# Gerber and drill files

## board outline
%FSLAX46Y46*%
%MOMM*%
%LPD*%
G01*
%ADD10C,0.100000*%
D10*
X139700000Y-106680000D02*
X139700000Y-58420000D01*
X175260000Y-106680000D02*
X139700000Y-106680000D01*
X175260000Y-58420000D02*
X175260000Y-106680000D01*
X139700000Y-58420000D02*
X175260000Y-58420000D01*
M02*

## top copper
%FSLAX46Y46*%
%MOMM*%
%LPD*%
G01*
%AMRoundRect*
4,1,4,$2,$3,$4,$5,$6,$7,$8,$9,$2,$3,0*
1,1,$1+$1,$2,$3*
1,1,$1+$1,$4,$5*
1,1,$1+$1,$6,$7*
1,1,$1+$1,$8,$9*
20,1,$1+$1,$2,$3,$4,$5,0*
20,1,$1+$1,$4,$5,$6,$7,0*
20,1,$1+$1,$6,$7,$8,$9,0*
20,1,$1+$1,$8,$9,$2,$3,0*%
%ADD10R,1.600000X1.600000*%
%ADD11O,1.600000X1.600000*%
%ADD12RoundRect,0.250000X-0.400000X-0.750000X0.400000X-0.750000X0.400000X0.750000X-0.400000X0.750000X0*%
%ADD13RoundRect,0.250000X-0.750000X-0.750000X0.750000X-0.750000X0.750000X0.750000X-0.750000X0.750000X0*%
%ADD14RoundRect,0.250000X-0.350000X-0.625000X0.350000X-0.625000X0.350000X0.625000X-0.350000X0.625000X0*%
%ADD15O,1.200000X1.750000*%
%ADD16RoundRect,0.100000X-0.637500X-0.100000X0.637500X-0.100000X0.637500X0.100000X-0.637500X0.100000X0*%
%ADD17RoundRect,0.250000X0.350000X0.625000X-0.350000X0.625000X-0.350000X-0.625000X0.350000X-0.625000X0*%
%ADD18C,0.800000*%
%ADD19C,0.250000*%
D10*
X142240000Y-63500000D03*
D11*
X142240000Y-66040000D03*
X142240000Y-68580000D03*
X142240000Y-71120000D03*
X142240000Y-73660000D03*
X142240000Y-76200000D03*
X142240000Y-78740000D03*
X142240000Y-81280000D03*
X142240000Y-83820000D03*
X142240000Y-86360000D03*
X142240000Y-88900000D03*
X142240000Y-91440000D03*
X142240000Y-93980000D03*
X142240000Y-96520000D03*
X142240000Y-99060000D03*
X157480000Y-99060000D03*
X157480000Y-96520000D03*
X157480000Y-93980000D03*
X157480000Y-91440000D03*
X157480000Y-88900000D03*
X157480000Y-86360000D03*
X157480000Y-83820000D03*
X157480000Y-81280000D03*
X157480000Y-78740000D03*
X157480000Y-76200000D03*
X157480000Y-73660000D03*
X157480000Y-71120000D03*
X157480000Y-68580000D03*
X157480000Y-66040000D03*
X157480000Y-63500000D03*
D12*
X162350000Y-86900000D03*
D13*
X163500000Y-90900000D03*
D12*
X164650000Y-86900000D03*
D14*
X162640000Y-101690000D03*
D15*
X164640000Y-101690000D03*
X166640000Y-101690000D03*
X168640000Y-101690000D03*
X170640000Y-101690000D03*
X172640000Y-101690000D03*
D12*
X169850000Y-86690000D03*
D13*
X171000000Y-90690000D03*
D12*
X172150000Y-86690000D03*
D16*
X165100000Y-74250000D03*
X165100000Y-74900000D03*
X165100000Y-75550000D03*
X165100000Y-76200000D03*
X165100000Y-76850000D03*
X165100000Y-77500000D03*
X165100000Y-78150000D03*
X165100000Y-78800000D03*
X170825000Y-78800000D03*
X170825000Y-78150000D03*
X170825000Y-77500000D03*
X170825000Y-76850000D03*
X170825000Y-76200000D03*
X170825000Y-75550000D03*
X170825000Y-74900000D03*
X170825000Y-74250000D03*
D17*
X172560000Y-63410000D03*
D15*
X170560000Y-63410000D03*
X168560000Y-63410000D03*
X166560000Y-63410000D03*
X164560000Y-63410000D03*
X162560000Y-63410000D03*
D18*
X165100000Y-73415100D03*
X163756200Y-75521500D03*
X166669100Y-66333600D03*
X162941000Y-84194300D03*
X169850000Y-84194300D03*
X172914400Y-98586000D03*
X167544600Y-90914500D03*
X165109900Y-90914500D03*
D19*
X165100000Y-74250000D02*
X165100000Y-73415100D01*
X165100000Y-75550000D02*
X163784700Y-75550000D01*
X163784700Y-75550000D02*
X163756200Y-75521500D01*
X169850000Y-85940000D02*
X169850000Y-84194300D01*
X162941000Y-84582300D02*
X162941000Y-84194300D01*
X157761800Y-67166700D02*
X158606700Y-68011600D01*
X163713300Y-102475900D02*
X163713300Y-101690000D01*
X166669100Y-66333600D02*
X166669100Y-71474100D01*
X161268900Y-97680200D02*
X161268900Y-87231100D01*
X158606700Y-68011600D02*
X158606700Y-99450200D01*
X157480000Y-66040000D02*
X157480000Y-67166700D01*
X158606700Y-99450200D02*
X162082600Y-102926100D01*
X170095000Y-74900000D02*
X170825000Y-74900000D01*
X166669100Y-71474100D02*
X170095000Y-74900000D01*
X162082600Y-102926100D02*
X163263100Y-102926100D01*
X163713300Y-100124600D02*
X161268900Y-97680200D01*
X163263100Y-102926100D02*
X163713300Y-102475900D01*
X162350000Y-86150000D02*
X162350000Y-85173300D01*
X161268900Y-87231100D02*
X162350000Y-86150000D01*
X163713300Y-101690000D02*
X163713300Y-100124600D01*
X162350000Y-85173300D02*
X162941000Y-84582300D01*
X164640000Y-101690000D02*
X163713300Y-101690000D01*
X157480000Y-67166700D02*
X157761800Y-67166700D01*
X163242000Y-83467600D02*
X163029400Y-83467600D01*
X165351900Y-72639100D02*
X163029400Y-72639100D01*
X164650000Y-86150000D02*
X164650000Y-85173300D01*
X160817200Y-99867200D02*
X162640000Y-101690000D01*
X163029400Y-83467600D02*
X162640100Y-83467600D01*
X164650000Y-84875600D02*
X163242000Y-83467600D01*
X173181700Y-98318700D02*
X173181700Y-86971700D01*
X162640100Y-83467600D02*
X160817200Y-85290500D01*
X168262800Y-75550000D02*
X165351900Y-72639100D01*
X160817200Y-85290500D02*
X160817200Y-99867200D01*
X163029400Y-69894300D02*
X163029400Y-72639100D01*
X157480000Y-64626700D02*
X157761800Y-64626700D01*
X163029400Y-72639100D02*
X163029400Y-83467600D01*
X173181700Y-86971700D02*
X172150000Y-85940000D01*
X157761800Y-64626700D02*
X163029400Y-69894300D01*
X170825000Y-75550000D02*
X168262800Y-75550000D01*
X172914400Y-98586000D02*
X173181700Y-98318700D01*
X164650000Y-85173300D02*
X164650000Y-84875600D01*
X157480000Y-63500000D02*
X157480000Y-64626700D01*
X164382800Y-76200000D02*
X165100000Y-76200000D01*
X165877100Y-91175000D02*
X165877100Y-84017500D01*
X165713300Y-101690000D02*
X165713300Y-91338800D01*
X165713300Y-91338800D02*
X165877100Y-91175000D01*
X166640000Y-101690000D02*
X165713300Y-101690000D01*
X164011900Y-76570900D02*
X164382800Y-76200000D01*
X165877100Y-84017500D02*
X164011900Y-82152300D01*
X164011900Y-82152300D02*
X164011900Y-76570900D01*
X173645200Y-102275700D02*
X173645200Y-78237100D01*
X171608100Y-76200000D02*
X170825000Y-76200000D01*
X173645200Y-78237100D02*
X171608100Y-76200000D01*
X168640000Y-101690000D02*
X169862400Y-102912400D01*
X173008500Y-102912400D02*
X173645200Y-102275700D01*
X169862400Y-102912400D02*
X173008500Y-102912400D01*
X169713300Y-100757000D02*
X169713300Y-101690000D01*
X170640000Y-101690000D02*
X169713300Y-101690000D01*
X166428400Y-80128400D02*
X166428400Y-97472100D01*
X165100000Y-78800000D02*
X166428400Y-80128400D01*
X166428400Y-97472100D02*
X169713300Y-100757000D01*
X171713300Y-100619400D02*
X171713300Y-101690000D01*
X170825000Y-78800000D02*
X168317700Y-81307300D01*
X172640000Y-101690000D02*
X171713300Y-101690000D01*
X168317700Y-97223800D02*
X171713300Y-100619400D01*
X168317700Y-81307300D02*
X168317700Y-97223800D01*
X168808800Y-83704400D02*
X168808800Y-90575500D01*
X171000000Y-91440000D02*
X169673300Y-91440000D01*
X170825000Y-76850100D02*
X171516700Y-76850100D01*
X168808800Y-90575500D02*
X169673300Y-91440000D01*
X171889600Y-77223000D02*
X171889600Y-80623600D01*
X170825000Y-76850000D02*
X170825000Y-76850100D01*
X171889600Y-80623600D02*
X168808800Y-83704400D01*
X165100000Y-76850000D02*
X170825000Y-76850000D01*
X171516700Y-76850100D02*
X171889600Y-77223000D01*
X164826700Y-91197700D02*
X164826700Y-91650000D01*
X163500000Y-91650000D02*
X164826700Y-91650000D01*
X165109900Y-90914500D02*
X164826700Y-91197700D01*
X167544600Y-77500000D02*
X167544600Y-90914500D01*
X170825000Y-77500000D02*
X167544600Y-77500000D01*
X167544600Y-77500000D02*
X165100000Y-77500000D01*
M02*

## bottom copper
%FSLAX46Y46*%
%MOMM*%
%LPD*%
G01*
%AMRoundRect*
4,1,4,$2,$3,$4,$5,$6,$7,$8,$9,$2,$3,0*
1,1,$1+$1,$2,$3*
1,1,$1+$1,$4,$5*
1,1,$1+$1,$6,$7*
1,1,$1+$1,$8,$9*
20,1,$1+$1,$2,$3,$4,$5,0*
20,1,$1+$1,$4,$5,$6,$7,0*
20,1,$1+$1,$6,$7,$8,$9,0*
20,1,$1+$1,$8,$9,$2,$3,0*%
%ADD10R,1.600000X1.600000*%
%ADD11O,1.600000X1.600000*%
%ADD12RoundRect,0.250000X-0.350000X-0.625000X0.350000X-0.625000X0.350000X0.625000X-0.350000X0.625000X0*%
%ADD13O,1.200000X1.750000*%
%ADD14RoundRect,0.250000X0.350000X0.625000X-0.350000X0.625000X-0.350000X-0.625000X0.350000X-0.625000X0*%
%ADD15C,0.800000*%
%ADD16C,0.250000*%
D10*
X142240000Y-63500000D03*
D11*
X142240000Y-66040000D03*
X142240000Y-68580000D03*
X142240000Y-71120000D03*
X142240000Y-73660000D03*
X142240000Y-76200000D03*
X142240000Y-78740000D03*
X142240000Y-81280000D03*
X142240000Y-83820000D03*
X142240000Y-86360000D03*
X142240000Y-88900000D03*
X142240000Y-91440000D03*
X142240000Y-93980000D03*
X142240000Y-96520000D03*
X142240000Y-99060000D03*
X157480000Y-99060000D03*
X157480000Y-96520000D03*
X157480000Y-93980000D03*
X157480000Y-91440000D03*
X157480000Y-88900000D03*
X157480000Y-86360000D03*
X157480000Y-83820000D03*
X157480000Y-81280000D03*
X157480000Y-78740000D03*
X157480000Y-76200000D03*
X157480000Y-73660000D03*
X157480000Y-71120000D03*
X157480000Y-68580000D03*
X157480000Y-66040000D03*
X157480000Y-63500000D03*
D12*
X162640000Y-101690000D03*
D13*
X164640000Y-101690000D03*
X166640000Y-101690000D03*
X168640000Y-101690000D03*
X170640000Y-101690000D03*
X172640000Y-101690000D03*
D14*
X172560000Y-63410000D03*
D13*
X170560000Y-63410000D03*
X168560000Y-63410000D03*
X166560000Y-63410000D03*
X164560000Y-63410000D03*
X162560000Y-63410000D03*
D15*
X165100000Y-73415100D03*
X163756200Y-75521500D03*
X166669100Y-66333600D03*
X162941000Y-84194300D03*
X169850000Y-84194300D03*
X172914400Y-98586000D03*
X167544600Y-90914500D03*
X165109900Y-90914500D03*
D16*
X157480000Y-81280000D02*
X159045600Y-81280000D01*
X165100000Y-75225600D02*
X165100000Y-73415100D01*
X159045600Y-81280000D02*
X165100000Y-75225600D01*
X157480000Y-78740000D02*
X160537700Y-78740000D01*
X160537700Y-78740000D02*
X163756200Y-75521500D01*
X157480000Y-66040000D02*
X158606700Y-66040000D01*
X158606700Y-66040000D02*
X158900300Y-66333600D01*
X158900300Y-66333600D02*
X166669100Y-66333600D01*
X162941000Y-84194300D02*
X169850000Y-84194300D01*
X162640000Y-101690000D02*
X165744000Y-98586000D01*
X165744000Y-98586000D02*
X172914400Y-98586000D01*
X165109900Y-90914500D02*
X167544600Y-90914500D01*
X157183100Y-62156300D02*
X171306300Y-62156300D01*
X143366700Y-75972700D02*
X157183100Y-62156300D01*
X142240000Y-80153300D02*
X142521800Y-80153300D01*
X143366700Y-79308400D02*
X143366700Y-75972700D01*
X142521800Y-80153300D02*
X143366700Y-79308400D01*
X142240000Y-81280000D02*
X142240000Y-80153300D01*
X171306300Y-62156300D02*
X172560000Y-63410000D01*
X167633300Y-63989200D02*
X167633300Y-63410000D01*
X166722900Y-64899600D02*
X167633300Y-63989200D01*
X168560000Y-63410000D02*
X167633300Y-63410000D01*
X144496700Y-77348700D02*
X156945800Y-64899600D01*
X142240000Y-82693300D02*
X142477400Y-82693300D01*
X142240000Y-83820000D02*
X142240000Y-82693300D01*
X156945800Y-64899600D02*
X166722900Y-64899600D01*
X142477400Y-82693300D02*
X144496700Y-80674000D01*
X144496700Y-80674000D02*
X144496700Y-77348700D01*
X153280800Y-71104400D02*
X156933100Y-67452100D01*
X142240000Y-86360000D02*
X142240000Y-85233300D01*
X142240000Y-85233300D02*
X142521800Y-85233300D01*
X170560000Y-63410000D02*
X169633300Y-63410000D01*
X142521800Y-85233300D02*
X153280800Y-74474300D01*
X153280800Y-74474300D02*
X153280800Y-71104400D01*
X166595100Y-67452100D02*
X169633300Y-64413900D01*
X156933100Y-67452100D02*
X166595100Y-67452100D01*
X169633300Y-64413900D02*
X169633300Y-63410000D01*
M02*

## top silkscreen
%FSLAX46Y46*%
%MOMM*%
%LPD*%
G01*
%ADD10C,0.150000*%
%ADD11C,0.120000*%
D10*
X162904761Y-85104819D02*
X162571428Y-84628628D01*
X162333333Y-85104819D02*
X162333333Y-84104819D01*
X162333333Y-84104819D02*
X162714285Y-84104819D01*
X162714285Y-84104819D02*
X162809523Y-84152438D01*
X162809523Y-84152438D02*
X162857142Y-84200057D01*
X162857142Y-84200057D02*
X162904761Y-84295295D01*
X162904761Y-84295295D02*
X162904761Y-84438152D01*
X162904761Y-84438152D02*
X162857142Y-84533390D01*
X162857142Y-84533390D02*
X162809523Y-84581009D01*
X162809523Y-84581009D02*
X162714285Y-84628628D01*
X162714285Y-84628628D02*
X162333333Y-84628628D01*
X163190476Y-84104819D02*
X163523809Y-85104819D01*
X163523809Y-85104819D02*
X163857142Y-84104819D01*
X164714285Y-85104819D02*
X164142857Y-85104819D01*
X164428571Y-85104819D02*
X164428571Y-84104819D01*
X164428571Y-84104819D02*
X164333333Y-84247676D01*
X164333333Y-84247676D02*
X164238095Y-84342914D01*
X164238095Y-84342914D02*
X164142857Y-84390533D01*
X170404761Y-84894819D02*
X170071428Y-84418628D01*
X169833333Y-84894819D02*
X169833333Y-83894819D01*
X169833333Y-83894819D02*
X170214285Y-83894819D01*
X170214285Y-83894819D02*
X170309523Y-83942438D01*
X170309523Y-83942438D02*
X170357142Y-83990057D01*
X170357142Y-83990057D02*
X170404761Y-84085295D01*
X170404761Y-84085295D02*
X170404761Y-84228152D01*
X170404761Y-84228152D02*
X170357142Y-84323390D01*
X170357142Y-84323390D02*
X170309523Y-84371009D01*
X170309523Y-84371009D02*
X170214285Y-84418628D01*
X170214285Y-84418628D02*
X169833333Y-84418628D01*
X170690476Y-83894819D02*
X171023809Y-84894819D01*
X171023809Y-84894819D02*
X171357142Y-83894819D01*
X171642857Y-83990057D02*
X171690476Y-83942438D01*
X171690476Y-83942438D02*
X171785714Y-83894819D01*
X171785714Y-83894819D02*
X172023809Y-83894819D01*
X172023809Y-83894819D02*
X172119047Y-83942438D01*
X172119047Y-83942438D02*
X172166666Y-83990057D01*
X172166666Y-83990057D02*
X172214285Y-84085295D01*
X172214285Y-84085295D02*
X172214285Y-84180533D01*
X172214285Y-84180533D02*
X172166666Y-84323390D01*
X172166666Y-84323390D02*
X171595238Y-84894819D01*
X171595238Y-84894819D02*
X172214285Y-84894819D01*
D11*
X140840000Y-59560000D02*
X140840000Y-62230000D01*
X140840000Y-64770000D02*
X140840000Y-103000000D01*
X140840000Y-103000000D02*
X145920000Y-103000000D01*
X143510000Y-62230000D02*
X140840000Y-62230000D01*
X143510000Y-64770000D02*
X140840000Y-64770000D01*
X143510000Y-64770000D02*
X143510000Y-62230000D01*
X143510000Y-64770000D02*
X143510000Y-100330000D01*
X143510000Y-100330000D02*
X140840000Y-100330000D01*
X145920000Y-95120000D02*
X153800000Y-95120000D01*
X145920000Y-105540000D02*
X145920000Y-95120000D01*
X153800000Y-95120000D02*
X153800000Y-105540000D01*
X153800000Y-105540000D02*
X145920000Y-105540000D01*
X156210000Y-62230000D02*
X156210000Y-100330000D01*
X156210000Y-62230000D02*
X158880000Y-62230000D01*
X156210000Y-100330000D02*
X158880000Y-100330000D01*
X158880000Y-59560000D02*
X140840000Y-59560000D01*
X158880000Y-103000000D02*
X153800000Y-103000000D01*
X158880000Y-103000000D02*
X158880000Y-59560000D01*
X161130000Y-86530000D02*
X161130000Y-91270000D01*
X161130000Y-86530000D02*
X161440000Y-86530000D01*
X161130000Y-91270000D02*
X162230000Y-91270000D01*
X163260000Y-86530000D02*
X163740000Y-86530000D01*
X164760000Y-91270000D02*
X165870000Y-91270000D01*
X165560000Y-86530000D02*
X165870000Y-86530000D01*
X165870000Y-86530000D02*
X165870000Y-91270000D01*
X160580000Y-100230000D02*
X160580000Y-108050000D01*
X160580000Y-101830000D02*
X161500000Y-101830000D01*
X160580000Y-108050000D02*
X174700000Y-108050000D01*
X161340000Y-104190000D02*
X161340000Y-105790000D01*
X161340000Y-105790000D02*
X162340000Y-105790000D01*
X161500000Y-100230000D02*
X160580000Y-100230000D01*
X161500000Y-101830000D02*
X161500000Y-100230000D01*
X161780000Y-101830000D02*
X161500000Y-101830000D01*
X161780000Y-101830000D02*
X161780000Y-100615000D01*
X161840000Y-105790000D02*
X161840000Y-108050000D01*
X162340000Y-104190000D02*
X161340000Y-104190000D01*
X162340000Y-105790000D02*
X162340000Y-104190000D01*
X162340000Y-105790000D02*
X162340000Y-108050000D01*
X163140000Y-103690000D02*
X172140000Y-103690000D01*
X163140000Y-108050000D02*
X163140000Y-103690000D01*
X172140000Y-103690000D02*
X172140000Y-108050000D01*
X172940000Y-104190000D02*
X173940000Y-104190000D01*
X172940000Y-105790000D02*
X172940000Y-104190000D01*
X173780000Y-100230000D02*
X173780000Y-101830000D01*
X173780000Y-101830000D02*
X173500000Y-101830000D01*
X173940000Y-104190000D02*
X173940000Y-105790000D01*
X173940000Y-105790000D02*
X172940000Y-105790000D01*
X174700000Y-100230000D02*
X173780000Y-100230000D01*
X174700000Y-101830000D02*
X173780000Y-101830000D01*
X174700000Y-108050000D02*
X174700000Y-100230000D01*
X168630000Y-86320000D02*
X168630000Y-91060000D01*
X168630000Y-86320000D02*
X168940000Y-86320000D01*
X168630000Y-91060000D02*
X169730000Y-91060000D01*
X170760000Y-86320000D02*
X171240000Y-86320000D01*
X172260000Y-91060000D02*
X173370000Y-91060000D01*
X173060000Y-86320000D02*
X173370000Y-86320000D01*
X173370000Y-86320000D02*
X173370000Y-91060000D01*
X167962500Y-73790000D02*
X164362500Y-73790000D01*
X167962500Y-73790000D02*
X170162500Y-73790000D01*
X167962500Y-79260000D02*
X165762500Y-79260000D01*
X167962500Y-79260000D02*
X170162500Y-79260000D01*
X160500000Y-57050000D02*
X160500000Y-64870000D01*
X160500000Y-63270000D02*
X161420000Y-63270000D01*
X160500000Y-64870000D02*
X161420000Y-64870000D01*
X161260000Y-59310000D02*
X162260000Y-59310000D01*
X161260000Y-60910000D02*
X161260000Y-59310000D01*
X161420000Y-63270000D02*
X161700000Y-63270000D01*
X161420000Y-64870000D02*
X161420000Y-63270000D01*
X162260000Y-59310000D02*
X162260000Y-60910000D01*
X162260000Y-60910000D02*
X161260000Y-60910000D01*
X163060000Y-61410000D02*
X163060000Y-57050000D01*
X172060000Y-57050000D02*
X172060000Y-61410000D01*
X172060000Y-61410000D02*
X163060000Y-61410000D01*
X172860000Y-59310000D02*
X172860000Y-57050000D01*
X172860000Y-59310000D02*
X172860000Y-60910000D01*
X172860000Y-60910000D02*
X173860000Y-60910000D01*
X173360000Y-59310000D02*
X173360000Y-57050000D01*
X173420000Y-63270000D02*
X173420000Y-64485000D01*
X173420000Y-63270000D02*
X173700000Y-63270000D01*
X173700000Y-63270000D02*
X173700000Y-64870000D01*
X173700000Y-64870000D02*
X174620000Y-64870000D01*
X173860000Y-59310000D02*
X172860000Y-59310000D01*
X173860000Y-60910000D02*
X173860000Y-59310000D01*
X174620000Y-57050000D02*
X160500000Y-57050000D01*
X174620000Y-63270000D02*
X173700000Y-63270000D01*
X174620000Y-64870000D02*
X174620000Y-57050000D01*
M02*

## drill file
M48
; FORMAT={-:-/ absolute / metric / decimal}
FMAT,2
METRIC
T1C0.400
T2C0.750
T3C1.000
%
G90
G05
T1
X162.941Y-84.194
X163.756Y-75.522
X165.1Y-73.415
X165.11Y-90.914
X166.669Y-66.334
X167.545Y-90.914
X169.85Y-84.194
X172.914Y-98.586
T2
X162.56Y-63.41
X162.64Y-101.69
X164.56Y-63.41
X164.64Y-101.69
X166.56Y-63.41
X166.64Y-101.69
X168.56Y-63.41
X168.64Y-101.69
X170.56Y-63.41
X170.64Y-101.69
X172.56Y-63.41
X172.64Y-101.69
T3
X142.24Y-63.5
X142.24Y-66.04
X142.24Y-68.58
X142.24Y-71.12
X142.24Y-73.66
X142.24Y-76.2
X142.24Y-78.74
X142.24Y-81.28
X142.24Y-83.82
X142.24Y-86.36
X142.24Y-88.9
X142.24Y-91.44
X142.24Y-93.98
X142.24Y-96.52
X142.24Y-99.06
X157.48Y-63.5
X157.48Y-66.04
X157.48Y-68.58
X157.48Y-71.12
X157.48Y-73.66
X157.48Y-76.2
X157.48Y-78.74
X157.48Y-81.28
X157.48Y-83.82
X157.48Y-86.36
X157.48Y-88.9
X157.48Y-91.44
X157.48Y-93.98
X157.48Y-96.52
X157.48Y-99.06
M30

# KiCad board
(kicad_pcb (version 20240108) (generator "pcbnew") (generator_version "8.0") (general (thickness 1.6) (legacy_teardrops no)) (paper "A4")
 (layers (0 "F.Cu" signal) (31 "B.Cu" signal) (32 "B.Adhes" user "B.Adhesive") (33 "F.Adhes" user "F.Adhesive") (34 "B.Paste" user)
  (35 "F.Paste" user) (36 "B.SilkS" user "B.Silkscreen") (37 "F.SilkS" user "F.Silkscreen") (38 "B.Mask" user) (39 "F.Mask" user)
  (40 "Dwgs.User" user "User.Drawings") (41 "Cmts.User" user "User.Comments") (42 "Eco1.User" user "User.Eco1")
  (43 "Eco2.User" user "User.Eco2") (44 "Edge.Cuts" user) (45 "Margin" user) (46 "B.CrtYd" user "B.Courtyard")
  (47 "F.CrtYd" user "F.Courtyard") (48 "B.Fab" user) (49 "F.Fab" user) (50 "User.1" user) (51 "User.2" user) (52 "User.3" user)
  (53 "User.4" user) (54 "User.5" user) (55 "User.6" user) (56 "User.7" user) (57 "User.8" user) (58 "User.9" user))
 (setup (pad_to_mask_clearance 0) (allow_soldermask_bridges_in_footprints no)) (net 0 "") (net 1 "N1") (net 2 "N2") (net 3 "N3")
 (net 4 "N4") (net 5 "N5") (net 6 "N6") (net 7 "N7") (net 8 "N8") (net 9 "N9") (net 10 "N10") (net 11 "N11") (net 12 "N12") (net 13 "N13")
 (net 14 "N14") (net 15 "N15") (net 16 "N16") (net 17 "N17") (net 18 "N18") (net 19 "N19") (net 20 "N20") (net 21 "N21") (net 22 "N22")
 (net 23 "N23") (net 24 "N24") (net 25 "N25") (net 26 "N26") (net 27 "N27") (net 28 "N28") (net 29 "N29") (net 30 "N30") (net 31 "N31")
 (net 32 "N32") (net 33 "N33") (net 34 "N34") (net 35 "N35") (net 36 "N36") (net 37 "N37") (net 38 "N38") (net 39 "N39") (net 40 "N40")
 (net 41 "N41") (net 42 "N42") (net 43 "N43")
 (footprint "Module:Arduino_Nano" (layer "F.Cu") (at 142.24 63.5)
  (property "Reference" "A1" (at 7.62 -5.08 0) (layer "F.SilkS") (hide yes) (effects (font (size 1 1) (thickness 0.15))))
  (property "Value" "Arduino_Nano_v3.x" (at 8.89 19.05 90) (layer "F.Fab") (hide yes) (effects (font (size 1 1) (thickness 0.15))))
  (fp_line (start -1.4 -3.94) (end -1.4 -1.27) (stroke (width 0.12) (type solid)) (layer "F.SilkS"))
  (fp_line (start -1.4 1.27) (end -1.4 39.5) (stroke (width 0.12) (type solid)) (layer "F.SilkS"))
  (fp_line (start -1.4 39.5) (end 3.68 39.5) (stroke (width 0.12) (type solid)) (layer "F.SilkS"))
  (fp_line (start 1.27 -1.27) (end -1.4 -1.27) (stroke (width 0.12) (type solid)) (layer "F.SilkS"))
  (fp_line (start 1.27 1.27) (end -1.4 1.27) (stroke (width 0.12) (type solid)) (layer "F.SilkS"))
  (fp_line (start 1.27 1.27) (end 1.27 -1.27) (stroke (width 0.12) (type solid)) (layer "F.SilkS"))
  (fp_line (start 1.27 1.27) (end 1.27 36.83) (stroke (width 0.12) (type solid)) (layer "F.SilkS"))
  (fp_line (start 1.27 36.83) (end -1.4 36.83) (stroke (width 0.12) (type solid)) (layer "F.SilkS"))
  (fp_line (start 3.68 31.62) (end 11.56 31.62) (stroke (width 0.12) (type solid)) (layer "F.SilkS"))
  (fp_line (start 3.68 42.04) (end 3.68 31.62) (stroke (width 0.12) (type solid)) (layer "F.SilkS"))
  (fp_line (start 11.56 31.62) (end 11.56 42.04) (stroke (width 0.12) (type solid)) (layer "F.SilkS"))
  (fp_line (start 11.56 42.04) (end 3.68 42.04) (stroke (width 0.12) (type solid)) (layer "F.SilkS"))
  (fp_line (start 13.97 -1.27) (end 13.97 36.83) (stroke (width 0.12) (type solid)) (layer "F.SilkS"))
  (fp_line (start 13.97 -1.27) (end 16.64 -1.27) (stroke (width 0.12) (type solid)) (layer "F.SilkS"))
  (fp_line (start 13.97 36.83) (end 16.64 36.83) (stroke (width 0.12) (type solid)) (layer "F.SilkS"))
  (fp_line (start 16.64 -3.94) (end -1.4 -3.94) (stroke (width 0.12) (type solid)) (layer "F.SilkS"))
  (fp_line (start 16.64 39.5) (end 11.56 39.5) (stroke (width 0.12) (type solid)) (layer "F.SilkS"))
  (fp_line (start 16.64 39.5) (end 16.64 -3.94) (stroke (width 0.12) (type solid)) (layer "F.SilkS"))
  (pad "1" thru_hole rect (at 0 0) (size 1.6 1.6) (drill 1) (layers "*.Cu" "*.Mask") (remove_unused_layers no) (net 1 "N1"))
  (pad "2" thru_hole oval (at 0 2.54) (size 1.6 1.6) (drill 1) (layers "*.Cu" "*.Mask") (remove_unused_layers no) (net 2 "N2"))
  (pad "3" thru_hole oval (at 0 5.08) (size 1.6 1.6) (drill 1) (layers "*.Cu" "*.Mask") (remove_unused_layers no) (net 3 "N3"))
  (pad "4" thru_hole oval (at 0 7.62) (size 1.6 1.6) (drill 1) (layers "*.Cu" "*.Mask") (remove_unused_layers no) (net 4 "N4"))
  (pad "5" thru_hole oval (at 0 10.16) (size 1.6 1.6) (drill 1) (layers "*.Cu" "*.Mask") (remove_unused_layers no) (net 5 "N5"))
  (pad "6" thru_hole oval (at 0 12.7) (size 1.6 1.6) (drill 1) (layers "*.Cu" "*.Mask") (remove_unused_layers no) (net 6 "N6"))
  (pad "7" thru_hole oval (at 0 15.24) (size 1.6 1.6) (drill 1) (layers "*.Cu" "*.Mask") (remove_unused_layers no) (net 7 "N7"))
  (pad "8" thru_hole oval (at 0 17.78) (size 1.6 1.6) (drill 1) (layers "*.Cu" "*.Mask") (remove_unused_layers no) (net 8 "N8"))
  (pad "9" thru_hole oval (at 0 20.32) (size 1.6 1.6) (drill 1) (layers "*.Cu" "*.Mask") (remove_unused_layers no) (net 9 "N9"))
  (pad "10" thru_hole oval (at 0 22.86) (size 1.6 1.6) (drill 1) (layers "*.Cu" "*.Mask") (remove_unused_layers no) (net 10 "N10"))
  (pad "11" thru_hole oval (at 0 25.4) (size 1.6 1.6) (drill 1) (layers "*.Cu" "*.Mask") (remove_unused_layers no) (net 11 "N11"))
  (pad "12" thru_hole oval (at 0 27.94) (size 1.6 1.6) (drill 1) (layers "*.Cu" "*.Mask") (remove_unused_layers no) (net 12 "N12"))
  (pad "13" thru_hole oval (at 0 30.48) (size 1.6 1.6) (drill 1) (layers "*.Cu" "*.Mask") (remove_unused_layers no) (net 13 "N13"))
  (pad "14" thru_hole oval (at 0 33.02) (size 1.6 1.6) (drill 1) (layers "*.Cu" "*.Mask") (remove_unused_layers no) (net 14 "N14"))
  (pad "15" thru_hole oval (at 0 35.56) (size 1.6 1.6) (drill 1) (layers "*.Cu" "*.Mask") (remove_unused_layers no) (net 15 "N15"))
  (pad "16" thru_hole oval (at 15.24 35.56) (size 1.6 1.6) (drill 1) (layers "*.Cu" "*.Mask") (remove_unused_layers no) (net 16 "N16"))
  (pad "17" thru_hole oval (at 15.24 33.02) (size 1.6 1.6) (drill 1) (layers "*.Cu" "*.Mask") (remove_unused_layers no) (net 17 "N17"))
  (pad "18" thru_hole oval (at 15.24 30.48) (size 1.6 1.6) (drill 1) (layers "*.Cu" "*.Mask") (remove_unused_layers no) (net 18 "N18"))
  (pad "19" thru_hole oval (at 15.24 27.94) (size 1.6 1.6) (drill 1) (layers "*.Cu" "*.Mask") (remove_unused_layers no) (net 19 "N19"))
  (pad "20" thru_hole oval (at 15.24 25.4) (size 1.6 1.6) (drill 1) (layers "*.Cu" "*.Mask") (remove_unused_layers no) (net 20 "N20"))
  (pad "21" thru_hole oval (at 15.24 22.86) (size 1.6 1.6) (drill 1) (layers "*.Cu" "*.Mask") (remove_unused_layers no) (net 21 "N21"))
  (pad "22" thru_hole oval (at 15.24 20.32) (size 1.6 1.6) (drill 1) (layers "*.Cu" "*.Mask") (remove_unused_layers no) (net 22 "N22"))
  (pad "23" thru_hole oval (at 15.24 17.78) (size 1.6 1.6) (drill 1) (layers "*.Cu" "*.Mask") (remove_unused_layers no) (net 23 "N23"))
  (pad "24" thru_hole oval (at 15.24 15.24) (size 1.6 1.6) (drill 1) (layers "*.Cu" "*.Mask") (remove_unused_layers no) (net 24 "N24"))
  (pad "25" thru_hole oval (at 15.24 12.7) (size 1.6 1.6) (drill 1) (layers "*.Cu" "*.Mask") (remove_unused_layers no) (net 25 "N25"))
  (pad "26" thru_hole oval (at 15.24 10.16) (size 1.6 1.6) (drill 1) (layers "*.Cu" "*.Mask") (remove_unused_layers no) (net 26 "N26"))
  (pad "27" thru_hole oval (at 15.24 7.62) (size 1.6 1.6) (drill 1) (layers "*.Cu" "*.Mask") (remove_unused_layers no) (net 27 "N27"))
  (pad "28" thru_hole oval (at 15.24 5.08) (size 1.6 1.6) (drill 1) (layers "*.Cu" "*.Mask") (remove_unused_layers no) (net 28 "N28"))
  (pad "29" thru_hole oval (at 15.24 2.54) (size 1.6 1.6) (drill 1) (layers "*.Cu" "*.Mask") (remove_unused_layers no) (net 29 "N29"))
  (pad "30" thru_hole oval (at 15.24 0) (size 1.6 1.6) (drill 1) (layers "*.Cu" "*.Mask") (remove_unused_layers no) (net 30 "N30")))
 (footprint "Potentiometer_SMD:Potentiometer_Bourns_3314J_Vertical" (layer "F.Cu") (at 163.5 88.9)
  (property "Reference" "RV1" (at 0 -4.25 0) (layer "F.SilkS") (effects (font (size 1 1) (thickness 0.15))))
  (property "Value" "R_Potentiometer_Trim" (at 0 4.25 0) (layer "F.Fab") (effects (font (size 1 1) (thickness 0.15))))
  (fp_line (start -2.37 -2.37) (end -2.37 2.37) (stroke (width 0.12) (type solid)) (layer "F.SilkS"))
  (fp_line (start -2.37 -2.37) (end -2.06 -2.37) (stroke (width 0.12) (type solid)) (layer "F.SilkS"))
  (fp_line (start -2.37 2.37) (end -1.27 2.37) (stroke (width 0.12) (type solid)) (layer "F.SilkS"))
  (fp_line (start -0.24 -2.37) (end 0.24 -2.37) (stroke (width 0.12) (type solid)) (layer "F.SilkS"))
  (fp_line (start 1.26 2.37) (end 2.37 2.37) (stroke (width 0.12) (type solid)) (layer "F.SilkS"))
  (fp_line (start 2.06 -2.37) (end 2.37 -2.37) (stroke (width 0.12) (type solid)) (layer "F.SilkS"))
  (fp_line (start 2.37 -2.37) (end 2.37 2.37) (stroke (width 0.12) (type solid)) (layer "F.SilkS"))
  (pad "1" smd roundrect (at -1.15 -2) (size 1.3 2) (layers "F.Cu" "F.Paste" "F.Mask") (roundrect_rratio 0.1923076923) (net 30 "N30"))
  (pad "2" smd roundrect (at 0 2) (size 2 2) (layers "F.Cu" "F.Paste" "F.Mask") (roundrect_rratio 0.125) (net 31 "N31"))
  (pad "3" smd roundrect (at 1.15 -2) (size 1.3 2) (layers "F.Cu" "F.Paste" "F.Mask") (roundrect_rratio 0.1923076923) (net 29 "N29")))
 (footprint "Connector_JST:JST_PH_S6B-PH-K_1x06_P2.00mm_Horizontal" (layer "F.Cu") (at 162.64 101.69)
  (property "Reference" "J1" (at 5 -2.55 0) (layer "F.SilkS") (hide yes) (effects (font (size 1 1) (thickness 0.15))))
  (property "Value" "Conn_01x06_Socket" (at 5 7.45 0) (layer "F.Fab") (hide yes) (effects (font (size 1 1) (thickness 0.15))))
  (fp_line (start -2.06 -1.46) (end -2.06 6.36) (stroke (width 0.12) (type solid)) (layer "F.SilkS"))
  (fp_line (start -2.06 0.14) (end -1.14 0.14) (stroke (width 0.12) (type solid)) (layer "F.SilkS"))
  (fp_line (start -2.06 6.36) (end 12.06 6.36) (stroke (width 0.12) (type solid)) (layer "F.SilkS"))
  (fp_line (start -1.3 2.5) (end -1.3 4.1) (stroke (width 0.12) (type solid)) (layer "F.SilkS"))
  (fp_line (start -1.3 4.1) (end -0.3 4.1) (stroke (width 0.12) (type solid)) (layer "F.SilkS"))
  (fp_line (start -1.14 -1.46) (end -2.06 -1.46) (stroke (width 0.12) (type solid)) (layer "F.SilkS"))
  (fp_line (start -1.14 0.14) (end -1.14 -1.46) (stroke (width 0.12) (type solid)) (layer "F.SilkS"))
  (fp_line (start -0.86 0.14) (end -1.14 0.14) (stroke (width 0.12) (type solid)) (layer "F.SilkS"))
  (fp_line (start -0.86 0.14) (end -0.86 -1.075) (stroke (width 0.12) (type solid)) (layer "F.SilkS"))
  (fp_line (start -0.8 4.1) (end -0.8 6.36) (stroke (width 0.12) (type solid)) (layer "F.SilkS"))
  (fp_line (start -0.3 2.5) (end -1.3 2.5) (stroke (width 0.12) (type solid)) (layer "F.SilkS"))
  (fp_line (start -0.3 4.1) (end -0.3 2.5) (stroke (width 0.12) (type solid)) (layer "F.SilkS"))
  (fp_line (start -0.3 4.1) (end -0.3 6.36) (stroke (width 0.12) (type solid)) (layer "F.SilkS"))
  (fp_line (start 0.5 2) (end 9.5 2) (stroke (width 0.12) (type solid)) (layer "F.SilkS"))
  (fp_line (start 0.5 6.36) (end 0.5 2) (stroke (width 0.12) (type solid)) (layer "F.SilkS"))
  (fp_line (start 9.5 2) (end 9.5 6.36) (stroke (width 0.12) (type solid)) (layer "F.SilkS"))
  (fp_line (start 10.3 2.5) (end 11.3 2.5) (stroke (width 0.12) (type solid)) (layer "F.SilkS"))
  (fp_line (start 10.3 4.1) (end 10.3 2.5) (stroke (width 0.12) (type solid)) (layer "F.SilkS"))
  (fp_line (start 11.14 -1.46) (end 11.14 0.14) (stroke (width 0.12) (type solid)) (layer "F.SilkS"))
  (fp_line (start 11.14 0.14) (end 10.86 0.14) (stroke (width 0.12) (type solid)) (layer "F.SilkS"))
  (fp_line (start 11.3 2.5) (end 11.3 4.1) (stroke (width 0.12) (type solid)) (layer "F.SilkS"))
  (fp_line (start 11.3 4.1) (end 10.3 4.1) (stroke (width 0.12) (type solid)) (layer "F.SilkS"))
  (fp_line (start 12.06 -1.46) (end 11.14 -1.46) (stroke (width 0.12) (type solid)) (layer "F.SilkS"))
  (fp_line (start 12.06 0.14) (end 11.14 0.14) (stroke (width 0.12) (type solid)) (layer "F.SilkS"))
  (fp_line (start 12.06 6.36) (end 12.06 -1.46) (stroke (width 0.12) (type solid)) (layer "F.SilkS"))
  (pad "1" thru_hole roundrect (at 0 0) (size 1.2 1.75) (drill 0.75) (layers "*.Cu" "*.Mask") (remove_unused_layers no)
   (roundrect_rratio 0.208333) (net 30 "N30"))
  (pad "2" thru_hole oval (at 2 0) (size 1.2 1.75) (drill 0.75) (layers "*.Cu" "*.Mask") (remove_unused_layers no) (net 29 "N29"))
  (pad "3" thru_hole oval (at 4 0) (size 1.2 1.75) (drill 0.75) (layers "*.Cu" "*.Mask") (remove_unused_layers no) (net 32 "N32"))
  (pad "4" thru_hole oval (at 6 0) (size 1.2 1.75) (drill 0.75) (layers "*.Cu" "*.Mask") (remove_unused_layers no) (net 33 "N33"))
  (pad "5" thru_hole oval (at 8 0) (size 1.2 1.75) (drill 0.75) (layers "*.Cu" "*.Mask") (remove_unused_layers no) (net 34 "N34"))
  (pad "6" thru_hole oval (at 10 0) (size 1.2 1.75) (drill 0.75) (layers "*.Cu" "*.Mask") (remove_unused_layers no) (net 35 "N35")))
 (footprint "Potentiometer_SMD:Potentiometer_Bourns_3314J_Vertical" (layer "F.Cu") (at 171 88.69)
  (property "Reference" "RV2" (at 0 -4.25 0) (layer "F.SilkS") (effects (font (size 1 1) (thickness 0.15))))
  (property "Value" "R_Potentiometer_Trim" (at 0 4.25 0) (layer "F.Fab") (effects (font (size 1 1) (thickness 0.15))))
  (fp_line (start -2.37 -2.37) (end -2.37 2.37) (stroke (width 0.12) (type solid)) (layer "F.SilkS"))
  (fp_line (start -2.37 -2.37) (end -2.06 -2.37) (stroke (width 0.12) (type solid)) (layer "F.SilkS"))
  (fp_line (start -2.37 2.37) (end -1.27 2.37) (stroke (width 0.12) (type solid)) (layer "F.SilkS"))
  (fp_line (start -0.24 -2.37) (end 0.24 -2.37) (stroke (width 0.12) (type solid)) (layer "F.SilkS"))
  (fp_line (start 1.26 2.37) (end 2.37 2.37) (stroke (width 0.12) (type solid)) (layer "F.SilkS"))
  (fp_line (start 2.06 -2.37) (end 2.37 -2.37) (stroke (width 0.12) (type solid)) (layer "F.SilkS"))
  (fp_line (start 2.37 -2.37) (end 2.37 2.37) (stroke (width 0.12) (type solid)) (layer "F.SilkS"))
  (pad "1" smd roundrect (at -1.15 -2) (size 1.3 2) (layers "F.Cu" "F.Paste" "F.Mask") (roundrect_rratio 0.1923076923) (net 30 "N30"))
  (pad "2" smd roundrect (at 0 2) (size 2 2) (layers "F.Cu" "F.Paste" "F.Mask") (roundrect_rratio 0.125) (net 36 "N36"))
  (pad "3" smd roundrect (at 1.15 -2) (size 1.3 2) (layers "F.Cu" "F.Paste" "F.Mask") (roundrect_rratio 0.1923076923) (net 29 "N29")))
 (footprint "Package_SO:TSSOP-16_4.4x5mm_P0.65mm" (layer "F.Cu") (at 167.9625 76.525)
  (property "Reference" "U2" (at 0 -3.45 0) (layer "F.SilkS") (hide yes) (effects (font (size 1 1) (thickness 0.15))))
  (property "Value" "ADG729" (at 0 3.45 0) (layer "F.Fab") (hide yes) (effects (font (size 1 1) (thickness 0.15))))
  (fp_line (start 0 -2.735) (end -3.6 -2.735) (stroke (width 0.12) (type solid)) (layer "F.SilkS"))
  (fp_line (start 0 -2.735) (end 2.2 -2.735) (stroke (width 0.12) (type solid)) (layer "F.SilkS"))
  (fp_line (start 0 2.735) (end -2.2 2.735) (stroke (width 0.12) (type solid)) (layer "F.SilkS"))
  (fp_line (start 0 2.735) (end 2.2 2.735) (stroke (width 0.12) (type solid)) (layer "F.SilkS"))
  (pad "1" smd roundrect (at -2.8625 -2.275) (size 1.475 0.4) (layers "F.Cu" "F.Paste" "F.Mask") (roundrect_rratio 0.25) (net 23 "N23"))
  (pad "2" smd roundrect (at -2.8625 -1.625) (size 1.475 0.4) (layers "F.Cu" "F.Paste" "F.Mask") (roundrect_rratio 0.25) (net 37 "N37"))
  (pad "3" smd roundrect (at -2.8625 -0.975) (size 1.475 0.4) (layers "F.Cu" "F.Paste" "F.Mask") (roundrect_rratio 0.25) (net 24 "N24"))
  (pad "4" smd roundrect (at -2.8625 -0.325) (size 1.475 0.4) (layers "F.Cu" "F.Paste" "F.Mask") (roundrect_rratio 0.25) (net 32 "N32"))
  (pad "5" smd roundrect (at -2.8625 0.325) (size 1.475 0.4) (layers "F.Cu" "F.Paste" "F.Mask") (roundrect_rratio 0.25) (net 36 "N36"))
  (pad "6" smd roundrect (at -2.8625 0.975) (size 1.475 0.4) (layers "F.Cu" "F.Paste" "F.Mask") (roundrect_rratio 0.25) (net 31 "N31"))
  (pad "7" smd roundrect (at -2.8625 1.625) (size 1.475 0.4) (layers "F.Cu" "F.Paste" "F.Mask") (roundrect_rratio 0.25) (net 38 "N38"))
  (pad "8" smd roundrect (at -2.8625 2.275) (size 1.475 0.4) (layers "F.Cu" "F.Paste" "F.Mask") (roundrect_rratio 0.25) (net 34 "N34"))
  (pad "9" smd roundrect (at 2.8625 2.275) (size 1.475 0.4) (layers "F.Cu" "F.Paste" "F.Mask") (roundrect_rratio 0.25) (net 35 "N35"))
  (pad "10" smd roundrect (at 2.8625 1.625) (size 1.475 0.4) (layers "F.Cu" "F.Paste" "F.Mask") (roundrect_rratio 0.25) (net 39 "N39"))
  (pad "11" smd roundrect (at 2.8625 0.975) (size 1.475 0.4) (layers "F.Cu" "F.Paste" "F.Mask") (roundrect_rratio 0.25) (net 31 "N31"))
  (pad "12" smd roundrect (at 2.8625 0.325) (size 1.475 0.4) (layers "F.Cu" "F.Paste" "F.Mask") (roundrect_rratio 0.25) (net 36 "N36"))
  (pad "13" smd roundrect (at 2.8625 -0.325) (size 1.475 0.4) (layers "F.Cu" "F.Paste" "F.Mask") (roundrect_rratio 0.25) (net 33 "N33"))
  (pad "14" smd roundrect (at 2.8625 -0.975) (size 1.475 0.4) (layers "F.Cu" "F.Paste" "F.Mask") (roundrect_rratio 0.25) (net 30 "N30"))
  (pad "15" smd roundrect (at 2.8625 -1.625) (size 1.475 0.4) (layers "F.Cu" "F.Paste" "F.Mask") (roundrect_rratio 0.25) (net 29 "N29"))
  (pad "16" smd roundrect (at 2.8625 -2.275) (size 1.475 0.4) (layers "F.Cu" "F.Paste" "F.Mask") (roundrect_rratio 0.25) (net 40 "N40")))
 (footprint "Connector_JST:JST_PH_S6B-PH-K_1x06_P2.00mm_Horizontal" (layer "F.Cu") (at 172.56 63.41 180)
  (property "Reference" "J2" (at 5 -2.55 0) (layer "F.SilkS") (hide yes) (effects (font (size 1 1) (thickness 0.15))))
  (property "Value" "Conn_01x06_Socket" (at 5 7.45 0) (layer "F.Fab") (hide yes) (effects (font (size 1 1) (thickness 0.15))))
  (fp_line (start 12.06 6.36) (end 12.06 -1.46) (stroke (width 0.12) (type solid)) (layer "F.SilkS"))
  (fp_line (start 12.06 0.14) (end 11.14 0.14) (stroke (width 0.12) (type solid)) (layer "F.SilkS"))
  (fp_line (start 12.06 -1.46) (end 11.14 -1.46) (stroke (width 0.12) (type solid)) (layer "F.SilkS"))
  (fp_line (start 11.3 4.1) (end 10.3 4.1) (stroke (width 0.12) (type solid)) (layer "F.SilkS"))
  (fp_line (start 11.3 2.5) (end 11.3 4.1) (stroke (width 0.12) (type solid)) (layer "F.SilkS"))
  (fp_line (start 11.14 0.14) (end 10.86 0.14) (stroke (width 0.12) (type solid)) (layer "F.SilkS"))
  (fp_line (start 11.14 -1.46) (end 11.14 0.14) (stroke (width 0.12) (type solid)) (layer "F.SilkS"))
  (fp_line (start 10.3 4.1) (end 10.3 2.5) (stroke (width 0.12) (type solid)) (layer "F.SilkS"))
  (fp_line (start 10.3 2.5) (end 11.3 2.5) (stroke (width 0.12) (type solid)) (layer "F.SilkS"))
  (fp_line (start 9.5 2) (end 9.5 6.36) (stroke (width 0.12) (type solid)) (layer "F.SilkS"))
  (fp_line (start 0.5 6.36) (end 0.5 2) (stroke (width 0.12) (type solid)) (layer "F.SilkS"))
  (fp_line (start 0.5 2) (end 9.5 2) (stroke (width 0.12) (type solid)) (layer "F.SilkS"))
  (fp_line (start -0.3 4.1) (end -0.3 6.36) (stroke (width 0.12) (type solid)) (layer "F.SilkS"))
  (fp_line (start -0.3 4.1) (end -0.3 2.5) (stroke (width 0.12) (type solid)) (layer "F.SilkS"))
  (fp_line (start -0.3 2.5) (end -1.3 2.5) (stroke (width 0.12) (type solid)) (layer "F.SilkS"))
  (fp_line (start -0.8 4.1) (end -0.8 6.36) (stroke (width 0.12) (type solid)) (layer "F.SilkS"))
  (fp_line (start -0.86 0.14) (end -0.86 -1.075) (stroke (width 0.12) (type solid)) (layer "F.SilkS"))
  (fp_line (start -0.86 0.14) (end -1.14 0.14) (stroke (width 0.12) (type solid)) (layer "F.SilkS"))
  (fp_line (start -1.14 0.14) (end -1.14 -1.46) (stroke (width 0.12) (type solid)) (layer "F.SilkS"))
  (fp_line (start -1.14 -1.46) (end -2.06 -1.46) (stroke (width 0.12) (type solid)) (layer "F.SilkS"))
  (fp_line (start -1.3 4.1) (end -0.3 4.1) (stroke (width 0.12) (type solid)) (layer "F.SilkS"))
  (fp_line (start -1.3 2.5) (end -1.3 4.1) (stroke (width 0.12) (type solid)) (layer "F.SilkS"))
  (fp_line (start -2.06 6.36) (end 12.06 6.36) (stroke (width 0.12) (type solid)) (layer "F.SilkS"))
  (fp_line (start -2.06 0.14) (end -1.14 0.14) (stroke (width 0.12) (type solid)) (layer "F.SilkS"))
  (fp_line (start -2.06 -1.46) (end -2.06 6.36) (stroke (width 0.12) (type solid)) (layer "F.SilkS"))
  (pad "1" thru_hole roundrect (at 0 0 180) (size 1.2 1.75) (drill 0.75) (layers "*.Cu" "*.Mask") (remove_unused_layers no)
   (roundrect_rratio 0.208333) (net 8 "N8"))
  (pad "2" thru_hole oval (at 2 0 180) (size 1.2 1.75) (drill 0.75) (layers "*.Cu" "*.Mask") (remove_unused_layers no) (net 10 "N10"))
  (pad "3" thru_hole oval (at 4 0 180) (size 1.2 1.75) (drill 0.75) (layers "*.Cu" "*.Mask") (remove_unused_layers no) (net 9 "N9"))
  (pad "4" thru_hole oval (at 6 0 180) (size 1.2 1.75) (drill 0.75) (layers "*.Cu" "*.Mask") (remove_unused_layers no) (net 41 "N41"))
  (pad "5" thru_hole oval (at 8 0 180) (size 1.2 1.75) (drill 0.75) (layers "*.Cu" "*.Mask") (remove_unused_layers no) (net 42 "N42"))
  (pad "6" thru_hole oval (at 10 0 180) (size 1.2 1.75) (drill 0.75) (layers "*.Cu" "*.Mask") (remove_unused_layers no) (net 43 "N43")))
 (gr_line (start 139.7 106.68) (end 139.7 58.42) (stroke (width 0.1) (type default)) (layer "Edge.Cuts"))
 (gr_line (start 175.26 106.68) (end 139.7 106.68) (stroke (width 0.1) (type default)) (layer "Edge.Cuts"))
 (gr_line (start 175.26 58.42) (end 175.26 106.68) (stroke (width 0.1) (type default)) (layer "Edge.Cuts"))
 (gr_line (start 139.7 58.42) (end 175.26 58.42) (stroke (width 0.1) (type default)) (layer "Edge.Cuts"))
 (segment (start 165.1 74.25) (end 165.1 73.4151) (width 0.25) (layer "F.Cu") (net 23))
 (via (at 165.1 73.4151) (size 0.8) (drill 0.4) (layers "F.Cu" "B.Cu") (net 23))
 (segment (start 157.48 81.28) (end 159.0456 81.28) (width 0.25) (layer "B.Cu") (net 23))
 (segment (start 165.1 75.2256) (end 165.1 73.4151) (width 0.25) (layer "B.Cu") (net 23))
 (segment (start 159.0456 81.28) (end 165.1 75.2256) (width 0.25) (layer "B.Cu") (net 23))
 (segment (start 165.1 75.55) (end 163.7847 75.55) (width 0.25) (layer "F.Cu") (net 24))
 (segment (start 163.7847 75.55) (end 163.7562 75.5215) (width 0.25) (layer "F.Cu") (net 24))
 (via (at 163.7562 75.5215) (size 0.8) (drill 0.4) (layers "F.Cu" "B.Cu") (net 24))
 (segment (start 157.48 78.74) (end 160.5377 78.74) (width 0.25) (layer "B.Cu") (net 24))
 (segment (start 160.5377 78.74) (end 163.7562 75.5215) (width 0.25) (layer "B.Cu") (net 24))
 (segment (start 169.85 85.94) (end 169.85 84.1943) (width 0.25) (layer "F.Cu") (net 29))
 (segment (start 162.941 84.5823) (end 162.941 84.1943) (width 0.25) (layer "F.Cu") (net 29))
 (segment (start 157.7618 67.1667) (end 158.6067 68.0116) (width 0.25) (layer "F.Cu") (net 29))
 (segment (start 163.7133 102.4759) (end 163.7133 101.69) (width 0.25) (layer "F.Cu") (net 29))
 (segment (start 166.6691 66.3336) (end 166.6691 71.4741) (width 0.25) (layer "F.Cu") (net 29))
 (segment (start 161.2689 97.6802) (end 161.2689 87.2311) (width 0.25) (layer "F.Cu") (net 29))
 (segment (start 158.6067 68.0116) (end 158.6067 99.4502) (width 0.25) (layer "F.Cu") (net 29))
 (segment (start 157.48 66.04) (end 157.48 67.1667) (width 0.25) (layer "F.Cu") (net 29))
 (segment (start 158.6067 99.4502) (end 162.0826 102.9261) (width 0.25) (layer "F.Cu") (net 29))
 (segment (start 170.095 74.9) (end 170.825 74.9) (width 0.25) (layer "F.Cu") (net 29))
 (segment (start 166.6691 71.4741) (end 170.095 74.9) (width 0.25) (layer "F.Cu") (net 29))
 (segment (start 162.0826 102.9261) (end 163.2631 102.9261) (width 0.25) (layer "F.Cu") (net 29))
 (segment (start 163.7133 100.1246) (end 161.2689 97.6802) (width 0.25) (layer "F.Cu") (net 29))
 (segment (start 163.2631 102.9261) (end 163.7133 102.4759) (width 0.25) (layer "F.Cu") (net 29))
 (segment (start 162.35 86.15) (end 162.35 85.1733) (width 0.25) (layer "F.Cu") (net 29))
 (segment (start 161.2689 87.2311) (end 162.35 86.15) (width 0.25) (layer "F.Cu") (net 29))
 (segment (start 163.7133 101.69) (end 163.7133 100.1246) (width 0.25) (layer "F.Cu") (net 29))
 (segment (start 162.35 85.1733) (end 162.941 84.5823) (width 0.25) (layer "F.Cu") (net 29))
 (segment (start 164.64 101.69) (end 163.7133 101.69) (width 0.25) (layer "F.Cu") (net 29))
 (segment (start 157.48 67.1667) (end 157.7618 67.1667) (width 0.25) (layer "F.Cu") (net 29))
 (via (at 166.6691 66.3336) (size 0.8) (drill 0.4) (layers "F.Cu" "B.Cu") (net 29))
 (via (at 162.941 84.1943) (size 0.8) (drill 0.4) (layers "F.Cu" "B.Cu") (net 29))
 (via (at 169.85 84.1943) (size 0.8) (drill 0.4) (layers "F.Cu" "B.Cu") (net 29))
 (segment (start 157.48 66.04) (end 158.6067 66.04) (width 0.25) (layer "B.Cu") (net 29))
 (segment (start 158.6067 66.04) (end 158.9003 66.3336) (width 0.25) (layer "B.Cu") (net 29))
 (segment (start 158.9003 66.3336) (end 166.6691 66.3336) (width 0.25) (layer "B.Cu") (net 29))
 (segment (start 162.941 84.1943) (end 169.85 84.1943) (width 0.25) (layer "B.Cu") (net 29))
 (segment (start 163.242 83.4676) (end 163.0294 83.4676) (width 0.25) (layer "F.Cu") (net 30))
 (segment (start 165.3519 72.6391) (end 163.0294 72.6391) (width 0.25) (layer "F.Cu") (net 30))
 (segment (start 164.65 86.15) (end 164.65 85.1733) (width 0.25) (layer "F.Cu") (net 30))
 (segment (start 160.8172 99.8672) (end 162.64 101.69) (width 0.25) (layer "F.Cu") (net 30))
 (segment (start 163.0294 83.4676) (end 162.6401 83.4676) (width 0.25) (layer "F.Cu") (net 30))
 (segment (start 164.65 84.8756) (end 163.242 83.4676) (width 0.25) (layer "F.Cu") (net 30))
 (segment (start 173.1817 98.3187) (end 173.1817 86.9717) (width 0.25) (layer "F.Cu") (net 30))
 (segment (start 162.6401 83.4676) (end 160.8172 85.2905) (width 0.25) (layer "F.Cu") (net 30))
 (segment (start 168.2628 75.55) (end 165.3519 72.6391) (width 0.25) (layer "F.Cu") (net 30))
 (segment (start 160.8172 85.2905) (end 160.8172 99.8672) (width 0.25) (layer "F.Cu") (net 30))
 (segment (start 163.0294 69.8943) (end 163.0294 72.6391) (width 0.25) (layer "F.Cu") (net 30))
 (segment (start 157.48 64.6267) (end 157.7618 64.6267) (width 0.25) (layer "F.Cu") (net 30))
 (segment (start 163.0294 72.6391) (end 163.0294 83.4676) (width 0.25) (layer "F.Cu") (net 30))
 (segment (start 173.1817 86.9717) (end 172.15 85.94) (width 0.25) (layer "F.Cu") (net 30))
 (segment (start 157.7618 64.6267) (end 163.0294 69.8943) (width 0.25) (layer "F.Cu") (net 30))
 (segment (start 170.825 75.55) (end 168.2628 75.55) (width 0.25) (layer "F.Cu") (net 30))
 (segment (start 172.9144 98.586) (end 173.1817 98.3187) (width 0.25) (layer "F.Cu") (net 30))
 (segment (start 164.65 85.1733) (end 164.65 84.8756) (width 0.25) (layer "F.Cu") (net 30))
 (segment (start 157.48 63.5) (end 157.48 64.6267) (width 0.25) (layer "F.Cu") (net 30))
 (via (at 172.9144 98.586) (size 0.8) (drill 0.4) (layers "F.Cu" "B.Cu") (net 30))
 (segment (start 162.64 101.69) (end 165.744 98.586) (width 0.25) (layer "B.Cu") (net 30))
 (segment (start 165.744 98.586) (end 172.9144 98.586) (width 0.25) (layer "B.Cu") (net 30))
 (segment (start 164.3828 76.2) (end 165.1 76.2) (width 0.25) (layer "F.Cu") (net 32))
 (segment (start 165.8771 91.175) (end 165.8771 84.0175) (width 0.25) (layer "F.Cu") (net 32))
 (segment (start 165.7133 101.69) (end 165.7133 91.3388) (width 0.25) (layer "F.Cu") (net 32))
 (segment (start 165.7133 91.3388) (end 165.8771 91.175) (width 0.25) (layer "F.Cu") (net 32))
 (segment (start 166.64 101.69) (end 165.7133 101.69) (width 0.25) (layer "F.Cu") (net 32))
 (segment (start 164.0119 76.5709) (end 164.3828 76.2) (width 0.25) (layer "F.Cu") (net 32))
 (segment (start 165.8771 84.0175) (end 164.0119 82.1523) (width 0.25) (layer "F.Cu") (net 32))
 (segment (start 164.0119 82.1523) (end 164.0119 76.5709) (width 0.25) (layer "F.Cu") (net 32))
 (segment (start 173.6452 102.2757) (end 173.6452 78.2371) (width 0.25) (layer "F.Cu") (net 33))
 (segment (start 171.6081 76.2) (end 170.825 76.2) (width 0.25) (layer "F.Cu") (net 33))
 (segment (start 173.6452 78.2371) (end 171.6081 76.2) (width 0.25) (layer "F.Cu") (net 33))
 (segment (start 168.64 101.69) (end 169.8624 102.9124) (width 0.25) (layer "F.Cu") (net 33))
 (segment (start 173.0085 102.9124) (end 173.6452 102.2757) (width 0.25) (layer "F.Cu") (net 33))
 (segment (start 169.8624 102.9124) (end 173.0085 102.9124) (width 0.25) (layer "F.Cu") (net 33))
 (segment (start 169.7133 100.757) (end 169.7133 101.69) (width 0.25) (layer "F.Cu") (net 34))
 (segment (start 170.64 101.69) (end 169.7133 101.69) (width 0.25) (layer "F.Cu") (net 34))
 (segment (start 166.4284 80.1284) (end 166.4284 97.4721) (width 0.25) (layer "F.Cu") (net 34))
 (segment (start 165.1 78.8) (end 166.4284 80.1284) (width 0.25) (layer "F.Cu") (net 34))
 (segment (start 166.4284 97.4721) (end 169.7133 100.757) (width 0.25) (layer "F.Cu") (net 34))
 (segment (start 171.7133 100.6194) (end 171.7133 101.69) (width 0.25) (layer "F.Cu") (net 35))
 (segment (start 170.825 78.8) (end 168.3177 81.3073) (width 0.25) (layer "F.Cu") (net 35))
 (segment (start 172.64 101.69) (end 171.7133 101.69) (width 0.25) (layer "F.Cu") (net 35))
 (segment (start 168.3177 97.2238) (end 171.7133 100.6194) (width 0.25) (layer "F.Cu") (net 35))
 (segment (start 168.3177 81.3073) (end 168.3177 97.2238) (width 0.25) (layer "F.Cu") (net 35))
 (segment (start 168.8088 83.7044) (end 168.8088 90.5755) (width 0.25) (layer "F.Cu") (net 36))
 (segment (start 171 91.44) (end 169.6733 91.44) (width 0.25) (layer "F.Cu") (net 36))
 (segment (start 170.825 76.8501) (end 171.5167 76.8501) (width 0.25) (layer "F.Cu") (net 36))
 (segment (start 168.8088 90.5755) (end 169.6733 91.44) (width 0.25) (layer "F.Cu") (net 36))
 (segment (start 171.8896 77.223) (end 171.8896 80.6236) (width 0.25) (layer "F.Cu") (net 36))
 (segment (start 170.825 76.85) (end 170.825 76.8501) (width 0.25) (layer "F.Cu") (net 36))
 (segment (start 171.8896 80.6236) (end 168.8088 83.7044) (width 0.25) (layer "F.Cu") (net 36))
 (segment (start 165.1 76.85) (end 170.825 76.85) (width 0.25) (layer "F.Cu") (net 36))
 (segment (start 171.5167 76.8501) (end 171.8896 77.223) (width 0.25) (layer "F.Cu") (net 36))
 (segment (start 164.8267 91.1977) (end 164.8267 91.65) (width 0.25) (layer "F.Cu") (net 31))
 (segment (start 163.5 91.65) (end 164.8267 91.65) (width 0.25) (layer "F.Cu") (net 31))
 (segment (start 165.1099 90.9145) (end 164.8267 91.1977) (width 0.25) (layer "F.Cu") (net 31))
 (segment (start 167.5446 77.5) (end 167.5446 90.9145) (width 0.25) (layer "F.Cu") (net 31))
 (segment (start 170.825 77.5) (end 167.5446 77.5) (width 0.25) (layer "F.Cu") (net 31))
 (segment (start 167.5446 77.5) (end 165.1 77.5) (width 0.25) (layer "F.Cu") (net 31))
 (via (at 167.5446 90.9145) (size 0.8) (drill 0.4) (layers "F.Cu" "B.Cu") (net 31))
 (via (at 165.1099 90.9145) (size 0.8) (drill 0.4) (layers "F.Cu" "B.Cu") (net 31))
 (segment (start 165.1099 90.9145) (end 167.5446 90.9145) (width 0.25) (layer "B.Cu") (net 31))
 (segment (start 157.1831 62.1563) (end 171.3063 62.1563) (width 0.25) (layer "B.Cu") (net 8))
 (segment (start 143.3667 75.9727) (end 157.1831 62.1563) (width 0.25) (layer "B.Cu") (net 8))
 (segment (start 142.24 80.1533) (end 142.5218 80.1533) (width 0.25) (layer "B.Cu") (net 8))
 (segment (start 143.3667 79.3084) (end 143.3667 75.9727) (width 0.25) (layer "B.Cu") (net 8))
 (segment (start 142.5218 80.1533) (end 143.3667 79.3084) (width 0.25) (layer "B.Cu") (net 8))
 (segment (start 142.24 81.28) (end 142.24 80.1533) (width 0.25) (layer "B.Cu") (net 8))
 (segment (start 171.3063 62.1563) (end 172.56 63.41) (width 0.25) (layer "B.Cu") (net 8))
 (segment (start 167.6333 63.9892) (end 167.6333 63.41) (width 0.25) (layer "B.Cu") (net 9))
 (segment (start 166.7229 64.8996) (end 167.6333 63.9892) (width 0.25) (layer "B.Cu") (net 9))
 (segment (start 168.56 63.41) (end 167.6333 63.41) (width 0.25) (layer "B.Cu") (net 9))
 (segment (start 144.4967 77.3487) (end 156.9458 64.8996) (width 0.25) (layer "B.Cu") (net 9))
 (segment (start 142.24 82.6933) (end 142.4774 82.6933) (width 0.25) (layer "B.Cu") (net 9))
 (segment (start 142.24 83.82) (end 142.24 82.6933) (width 0.25) (layer "B.Cu") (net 9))
 (segment (start 156.9458 64.8996) (end 166.7229 64.8996) (width 0.25) (layer "B.Cu") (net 9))
 (segment (start 142.4774 82.6933) (end 144.4967 80.674) (width 0.25) (layer "B.Cu") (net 9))
 (segment (start 144.4967 80.674) (end 144.4967 77.3487) (width 0.25) (layer "B.Cu") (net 9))
 (segment (start 153.2808 71.1044) (end 156.9331 67.4521) (width 0.25) (layer "B.Cu") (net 10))
 (segment (start 142.24 86.36) (end 142.24 85.2333) (width 0.25) (layer "B.Cu") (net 10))
 (segment (start 142.24 85.2333) (end 142.5218 85.2333) (width 0.25) (layer "B.Cu") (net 10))
 (segment (start 170.56 63.41) (end 169.6333 63.41) (width 0.25) (layer "B.Cu") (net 10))
 (segment (start 142.5218 85.2333) (end 153.2808 74.4743) (width 0.25) (layer "B.Cu") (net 10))
 (segment (start 153.2808 74.4743) (end 153.2808 71.1044) (width 0.25) (layer "B.Cu") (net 10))
 (segment (start 166.5951 67.4521) (end 169.6333 64.4139) (width 0.25) (layer "B.Cu") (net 10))
 (segment (start 156.9331 67.4521) (end 166.5951 67.4521) (width 0.25) (layer "B.Cu") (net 10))
 (segment (start 169.6333 64.4139) (end 169.6333 63.41) (width 0.25) (layer "B.Cu") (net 10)))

